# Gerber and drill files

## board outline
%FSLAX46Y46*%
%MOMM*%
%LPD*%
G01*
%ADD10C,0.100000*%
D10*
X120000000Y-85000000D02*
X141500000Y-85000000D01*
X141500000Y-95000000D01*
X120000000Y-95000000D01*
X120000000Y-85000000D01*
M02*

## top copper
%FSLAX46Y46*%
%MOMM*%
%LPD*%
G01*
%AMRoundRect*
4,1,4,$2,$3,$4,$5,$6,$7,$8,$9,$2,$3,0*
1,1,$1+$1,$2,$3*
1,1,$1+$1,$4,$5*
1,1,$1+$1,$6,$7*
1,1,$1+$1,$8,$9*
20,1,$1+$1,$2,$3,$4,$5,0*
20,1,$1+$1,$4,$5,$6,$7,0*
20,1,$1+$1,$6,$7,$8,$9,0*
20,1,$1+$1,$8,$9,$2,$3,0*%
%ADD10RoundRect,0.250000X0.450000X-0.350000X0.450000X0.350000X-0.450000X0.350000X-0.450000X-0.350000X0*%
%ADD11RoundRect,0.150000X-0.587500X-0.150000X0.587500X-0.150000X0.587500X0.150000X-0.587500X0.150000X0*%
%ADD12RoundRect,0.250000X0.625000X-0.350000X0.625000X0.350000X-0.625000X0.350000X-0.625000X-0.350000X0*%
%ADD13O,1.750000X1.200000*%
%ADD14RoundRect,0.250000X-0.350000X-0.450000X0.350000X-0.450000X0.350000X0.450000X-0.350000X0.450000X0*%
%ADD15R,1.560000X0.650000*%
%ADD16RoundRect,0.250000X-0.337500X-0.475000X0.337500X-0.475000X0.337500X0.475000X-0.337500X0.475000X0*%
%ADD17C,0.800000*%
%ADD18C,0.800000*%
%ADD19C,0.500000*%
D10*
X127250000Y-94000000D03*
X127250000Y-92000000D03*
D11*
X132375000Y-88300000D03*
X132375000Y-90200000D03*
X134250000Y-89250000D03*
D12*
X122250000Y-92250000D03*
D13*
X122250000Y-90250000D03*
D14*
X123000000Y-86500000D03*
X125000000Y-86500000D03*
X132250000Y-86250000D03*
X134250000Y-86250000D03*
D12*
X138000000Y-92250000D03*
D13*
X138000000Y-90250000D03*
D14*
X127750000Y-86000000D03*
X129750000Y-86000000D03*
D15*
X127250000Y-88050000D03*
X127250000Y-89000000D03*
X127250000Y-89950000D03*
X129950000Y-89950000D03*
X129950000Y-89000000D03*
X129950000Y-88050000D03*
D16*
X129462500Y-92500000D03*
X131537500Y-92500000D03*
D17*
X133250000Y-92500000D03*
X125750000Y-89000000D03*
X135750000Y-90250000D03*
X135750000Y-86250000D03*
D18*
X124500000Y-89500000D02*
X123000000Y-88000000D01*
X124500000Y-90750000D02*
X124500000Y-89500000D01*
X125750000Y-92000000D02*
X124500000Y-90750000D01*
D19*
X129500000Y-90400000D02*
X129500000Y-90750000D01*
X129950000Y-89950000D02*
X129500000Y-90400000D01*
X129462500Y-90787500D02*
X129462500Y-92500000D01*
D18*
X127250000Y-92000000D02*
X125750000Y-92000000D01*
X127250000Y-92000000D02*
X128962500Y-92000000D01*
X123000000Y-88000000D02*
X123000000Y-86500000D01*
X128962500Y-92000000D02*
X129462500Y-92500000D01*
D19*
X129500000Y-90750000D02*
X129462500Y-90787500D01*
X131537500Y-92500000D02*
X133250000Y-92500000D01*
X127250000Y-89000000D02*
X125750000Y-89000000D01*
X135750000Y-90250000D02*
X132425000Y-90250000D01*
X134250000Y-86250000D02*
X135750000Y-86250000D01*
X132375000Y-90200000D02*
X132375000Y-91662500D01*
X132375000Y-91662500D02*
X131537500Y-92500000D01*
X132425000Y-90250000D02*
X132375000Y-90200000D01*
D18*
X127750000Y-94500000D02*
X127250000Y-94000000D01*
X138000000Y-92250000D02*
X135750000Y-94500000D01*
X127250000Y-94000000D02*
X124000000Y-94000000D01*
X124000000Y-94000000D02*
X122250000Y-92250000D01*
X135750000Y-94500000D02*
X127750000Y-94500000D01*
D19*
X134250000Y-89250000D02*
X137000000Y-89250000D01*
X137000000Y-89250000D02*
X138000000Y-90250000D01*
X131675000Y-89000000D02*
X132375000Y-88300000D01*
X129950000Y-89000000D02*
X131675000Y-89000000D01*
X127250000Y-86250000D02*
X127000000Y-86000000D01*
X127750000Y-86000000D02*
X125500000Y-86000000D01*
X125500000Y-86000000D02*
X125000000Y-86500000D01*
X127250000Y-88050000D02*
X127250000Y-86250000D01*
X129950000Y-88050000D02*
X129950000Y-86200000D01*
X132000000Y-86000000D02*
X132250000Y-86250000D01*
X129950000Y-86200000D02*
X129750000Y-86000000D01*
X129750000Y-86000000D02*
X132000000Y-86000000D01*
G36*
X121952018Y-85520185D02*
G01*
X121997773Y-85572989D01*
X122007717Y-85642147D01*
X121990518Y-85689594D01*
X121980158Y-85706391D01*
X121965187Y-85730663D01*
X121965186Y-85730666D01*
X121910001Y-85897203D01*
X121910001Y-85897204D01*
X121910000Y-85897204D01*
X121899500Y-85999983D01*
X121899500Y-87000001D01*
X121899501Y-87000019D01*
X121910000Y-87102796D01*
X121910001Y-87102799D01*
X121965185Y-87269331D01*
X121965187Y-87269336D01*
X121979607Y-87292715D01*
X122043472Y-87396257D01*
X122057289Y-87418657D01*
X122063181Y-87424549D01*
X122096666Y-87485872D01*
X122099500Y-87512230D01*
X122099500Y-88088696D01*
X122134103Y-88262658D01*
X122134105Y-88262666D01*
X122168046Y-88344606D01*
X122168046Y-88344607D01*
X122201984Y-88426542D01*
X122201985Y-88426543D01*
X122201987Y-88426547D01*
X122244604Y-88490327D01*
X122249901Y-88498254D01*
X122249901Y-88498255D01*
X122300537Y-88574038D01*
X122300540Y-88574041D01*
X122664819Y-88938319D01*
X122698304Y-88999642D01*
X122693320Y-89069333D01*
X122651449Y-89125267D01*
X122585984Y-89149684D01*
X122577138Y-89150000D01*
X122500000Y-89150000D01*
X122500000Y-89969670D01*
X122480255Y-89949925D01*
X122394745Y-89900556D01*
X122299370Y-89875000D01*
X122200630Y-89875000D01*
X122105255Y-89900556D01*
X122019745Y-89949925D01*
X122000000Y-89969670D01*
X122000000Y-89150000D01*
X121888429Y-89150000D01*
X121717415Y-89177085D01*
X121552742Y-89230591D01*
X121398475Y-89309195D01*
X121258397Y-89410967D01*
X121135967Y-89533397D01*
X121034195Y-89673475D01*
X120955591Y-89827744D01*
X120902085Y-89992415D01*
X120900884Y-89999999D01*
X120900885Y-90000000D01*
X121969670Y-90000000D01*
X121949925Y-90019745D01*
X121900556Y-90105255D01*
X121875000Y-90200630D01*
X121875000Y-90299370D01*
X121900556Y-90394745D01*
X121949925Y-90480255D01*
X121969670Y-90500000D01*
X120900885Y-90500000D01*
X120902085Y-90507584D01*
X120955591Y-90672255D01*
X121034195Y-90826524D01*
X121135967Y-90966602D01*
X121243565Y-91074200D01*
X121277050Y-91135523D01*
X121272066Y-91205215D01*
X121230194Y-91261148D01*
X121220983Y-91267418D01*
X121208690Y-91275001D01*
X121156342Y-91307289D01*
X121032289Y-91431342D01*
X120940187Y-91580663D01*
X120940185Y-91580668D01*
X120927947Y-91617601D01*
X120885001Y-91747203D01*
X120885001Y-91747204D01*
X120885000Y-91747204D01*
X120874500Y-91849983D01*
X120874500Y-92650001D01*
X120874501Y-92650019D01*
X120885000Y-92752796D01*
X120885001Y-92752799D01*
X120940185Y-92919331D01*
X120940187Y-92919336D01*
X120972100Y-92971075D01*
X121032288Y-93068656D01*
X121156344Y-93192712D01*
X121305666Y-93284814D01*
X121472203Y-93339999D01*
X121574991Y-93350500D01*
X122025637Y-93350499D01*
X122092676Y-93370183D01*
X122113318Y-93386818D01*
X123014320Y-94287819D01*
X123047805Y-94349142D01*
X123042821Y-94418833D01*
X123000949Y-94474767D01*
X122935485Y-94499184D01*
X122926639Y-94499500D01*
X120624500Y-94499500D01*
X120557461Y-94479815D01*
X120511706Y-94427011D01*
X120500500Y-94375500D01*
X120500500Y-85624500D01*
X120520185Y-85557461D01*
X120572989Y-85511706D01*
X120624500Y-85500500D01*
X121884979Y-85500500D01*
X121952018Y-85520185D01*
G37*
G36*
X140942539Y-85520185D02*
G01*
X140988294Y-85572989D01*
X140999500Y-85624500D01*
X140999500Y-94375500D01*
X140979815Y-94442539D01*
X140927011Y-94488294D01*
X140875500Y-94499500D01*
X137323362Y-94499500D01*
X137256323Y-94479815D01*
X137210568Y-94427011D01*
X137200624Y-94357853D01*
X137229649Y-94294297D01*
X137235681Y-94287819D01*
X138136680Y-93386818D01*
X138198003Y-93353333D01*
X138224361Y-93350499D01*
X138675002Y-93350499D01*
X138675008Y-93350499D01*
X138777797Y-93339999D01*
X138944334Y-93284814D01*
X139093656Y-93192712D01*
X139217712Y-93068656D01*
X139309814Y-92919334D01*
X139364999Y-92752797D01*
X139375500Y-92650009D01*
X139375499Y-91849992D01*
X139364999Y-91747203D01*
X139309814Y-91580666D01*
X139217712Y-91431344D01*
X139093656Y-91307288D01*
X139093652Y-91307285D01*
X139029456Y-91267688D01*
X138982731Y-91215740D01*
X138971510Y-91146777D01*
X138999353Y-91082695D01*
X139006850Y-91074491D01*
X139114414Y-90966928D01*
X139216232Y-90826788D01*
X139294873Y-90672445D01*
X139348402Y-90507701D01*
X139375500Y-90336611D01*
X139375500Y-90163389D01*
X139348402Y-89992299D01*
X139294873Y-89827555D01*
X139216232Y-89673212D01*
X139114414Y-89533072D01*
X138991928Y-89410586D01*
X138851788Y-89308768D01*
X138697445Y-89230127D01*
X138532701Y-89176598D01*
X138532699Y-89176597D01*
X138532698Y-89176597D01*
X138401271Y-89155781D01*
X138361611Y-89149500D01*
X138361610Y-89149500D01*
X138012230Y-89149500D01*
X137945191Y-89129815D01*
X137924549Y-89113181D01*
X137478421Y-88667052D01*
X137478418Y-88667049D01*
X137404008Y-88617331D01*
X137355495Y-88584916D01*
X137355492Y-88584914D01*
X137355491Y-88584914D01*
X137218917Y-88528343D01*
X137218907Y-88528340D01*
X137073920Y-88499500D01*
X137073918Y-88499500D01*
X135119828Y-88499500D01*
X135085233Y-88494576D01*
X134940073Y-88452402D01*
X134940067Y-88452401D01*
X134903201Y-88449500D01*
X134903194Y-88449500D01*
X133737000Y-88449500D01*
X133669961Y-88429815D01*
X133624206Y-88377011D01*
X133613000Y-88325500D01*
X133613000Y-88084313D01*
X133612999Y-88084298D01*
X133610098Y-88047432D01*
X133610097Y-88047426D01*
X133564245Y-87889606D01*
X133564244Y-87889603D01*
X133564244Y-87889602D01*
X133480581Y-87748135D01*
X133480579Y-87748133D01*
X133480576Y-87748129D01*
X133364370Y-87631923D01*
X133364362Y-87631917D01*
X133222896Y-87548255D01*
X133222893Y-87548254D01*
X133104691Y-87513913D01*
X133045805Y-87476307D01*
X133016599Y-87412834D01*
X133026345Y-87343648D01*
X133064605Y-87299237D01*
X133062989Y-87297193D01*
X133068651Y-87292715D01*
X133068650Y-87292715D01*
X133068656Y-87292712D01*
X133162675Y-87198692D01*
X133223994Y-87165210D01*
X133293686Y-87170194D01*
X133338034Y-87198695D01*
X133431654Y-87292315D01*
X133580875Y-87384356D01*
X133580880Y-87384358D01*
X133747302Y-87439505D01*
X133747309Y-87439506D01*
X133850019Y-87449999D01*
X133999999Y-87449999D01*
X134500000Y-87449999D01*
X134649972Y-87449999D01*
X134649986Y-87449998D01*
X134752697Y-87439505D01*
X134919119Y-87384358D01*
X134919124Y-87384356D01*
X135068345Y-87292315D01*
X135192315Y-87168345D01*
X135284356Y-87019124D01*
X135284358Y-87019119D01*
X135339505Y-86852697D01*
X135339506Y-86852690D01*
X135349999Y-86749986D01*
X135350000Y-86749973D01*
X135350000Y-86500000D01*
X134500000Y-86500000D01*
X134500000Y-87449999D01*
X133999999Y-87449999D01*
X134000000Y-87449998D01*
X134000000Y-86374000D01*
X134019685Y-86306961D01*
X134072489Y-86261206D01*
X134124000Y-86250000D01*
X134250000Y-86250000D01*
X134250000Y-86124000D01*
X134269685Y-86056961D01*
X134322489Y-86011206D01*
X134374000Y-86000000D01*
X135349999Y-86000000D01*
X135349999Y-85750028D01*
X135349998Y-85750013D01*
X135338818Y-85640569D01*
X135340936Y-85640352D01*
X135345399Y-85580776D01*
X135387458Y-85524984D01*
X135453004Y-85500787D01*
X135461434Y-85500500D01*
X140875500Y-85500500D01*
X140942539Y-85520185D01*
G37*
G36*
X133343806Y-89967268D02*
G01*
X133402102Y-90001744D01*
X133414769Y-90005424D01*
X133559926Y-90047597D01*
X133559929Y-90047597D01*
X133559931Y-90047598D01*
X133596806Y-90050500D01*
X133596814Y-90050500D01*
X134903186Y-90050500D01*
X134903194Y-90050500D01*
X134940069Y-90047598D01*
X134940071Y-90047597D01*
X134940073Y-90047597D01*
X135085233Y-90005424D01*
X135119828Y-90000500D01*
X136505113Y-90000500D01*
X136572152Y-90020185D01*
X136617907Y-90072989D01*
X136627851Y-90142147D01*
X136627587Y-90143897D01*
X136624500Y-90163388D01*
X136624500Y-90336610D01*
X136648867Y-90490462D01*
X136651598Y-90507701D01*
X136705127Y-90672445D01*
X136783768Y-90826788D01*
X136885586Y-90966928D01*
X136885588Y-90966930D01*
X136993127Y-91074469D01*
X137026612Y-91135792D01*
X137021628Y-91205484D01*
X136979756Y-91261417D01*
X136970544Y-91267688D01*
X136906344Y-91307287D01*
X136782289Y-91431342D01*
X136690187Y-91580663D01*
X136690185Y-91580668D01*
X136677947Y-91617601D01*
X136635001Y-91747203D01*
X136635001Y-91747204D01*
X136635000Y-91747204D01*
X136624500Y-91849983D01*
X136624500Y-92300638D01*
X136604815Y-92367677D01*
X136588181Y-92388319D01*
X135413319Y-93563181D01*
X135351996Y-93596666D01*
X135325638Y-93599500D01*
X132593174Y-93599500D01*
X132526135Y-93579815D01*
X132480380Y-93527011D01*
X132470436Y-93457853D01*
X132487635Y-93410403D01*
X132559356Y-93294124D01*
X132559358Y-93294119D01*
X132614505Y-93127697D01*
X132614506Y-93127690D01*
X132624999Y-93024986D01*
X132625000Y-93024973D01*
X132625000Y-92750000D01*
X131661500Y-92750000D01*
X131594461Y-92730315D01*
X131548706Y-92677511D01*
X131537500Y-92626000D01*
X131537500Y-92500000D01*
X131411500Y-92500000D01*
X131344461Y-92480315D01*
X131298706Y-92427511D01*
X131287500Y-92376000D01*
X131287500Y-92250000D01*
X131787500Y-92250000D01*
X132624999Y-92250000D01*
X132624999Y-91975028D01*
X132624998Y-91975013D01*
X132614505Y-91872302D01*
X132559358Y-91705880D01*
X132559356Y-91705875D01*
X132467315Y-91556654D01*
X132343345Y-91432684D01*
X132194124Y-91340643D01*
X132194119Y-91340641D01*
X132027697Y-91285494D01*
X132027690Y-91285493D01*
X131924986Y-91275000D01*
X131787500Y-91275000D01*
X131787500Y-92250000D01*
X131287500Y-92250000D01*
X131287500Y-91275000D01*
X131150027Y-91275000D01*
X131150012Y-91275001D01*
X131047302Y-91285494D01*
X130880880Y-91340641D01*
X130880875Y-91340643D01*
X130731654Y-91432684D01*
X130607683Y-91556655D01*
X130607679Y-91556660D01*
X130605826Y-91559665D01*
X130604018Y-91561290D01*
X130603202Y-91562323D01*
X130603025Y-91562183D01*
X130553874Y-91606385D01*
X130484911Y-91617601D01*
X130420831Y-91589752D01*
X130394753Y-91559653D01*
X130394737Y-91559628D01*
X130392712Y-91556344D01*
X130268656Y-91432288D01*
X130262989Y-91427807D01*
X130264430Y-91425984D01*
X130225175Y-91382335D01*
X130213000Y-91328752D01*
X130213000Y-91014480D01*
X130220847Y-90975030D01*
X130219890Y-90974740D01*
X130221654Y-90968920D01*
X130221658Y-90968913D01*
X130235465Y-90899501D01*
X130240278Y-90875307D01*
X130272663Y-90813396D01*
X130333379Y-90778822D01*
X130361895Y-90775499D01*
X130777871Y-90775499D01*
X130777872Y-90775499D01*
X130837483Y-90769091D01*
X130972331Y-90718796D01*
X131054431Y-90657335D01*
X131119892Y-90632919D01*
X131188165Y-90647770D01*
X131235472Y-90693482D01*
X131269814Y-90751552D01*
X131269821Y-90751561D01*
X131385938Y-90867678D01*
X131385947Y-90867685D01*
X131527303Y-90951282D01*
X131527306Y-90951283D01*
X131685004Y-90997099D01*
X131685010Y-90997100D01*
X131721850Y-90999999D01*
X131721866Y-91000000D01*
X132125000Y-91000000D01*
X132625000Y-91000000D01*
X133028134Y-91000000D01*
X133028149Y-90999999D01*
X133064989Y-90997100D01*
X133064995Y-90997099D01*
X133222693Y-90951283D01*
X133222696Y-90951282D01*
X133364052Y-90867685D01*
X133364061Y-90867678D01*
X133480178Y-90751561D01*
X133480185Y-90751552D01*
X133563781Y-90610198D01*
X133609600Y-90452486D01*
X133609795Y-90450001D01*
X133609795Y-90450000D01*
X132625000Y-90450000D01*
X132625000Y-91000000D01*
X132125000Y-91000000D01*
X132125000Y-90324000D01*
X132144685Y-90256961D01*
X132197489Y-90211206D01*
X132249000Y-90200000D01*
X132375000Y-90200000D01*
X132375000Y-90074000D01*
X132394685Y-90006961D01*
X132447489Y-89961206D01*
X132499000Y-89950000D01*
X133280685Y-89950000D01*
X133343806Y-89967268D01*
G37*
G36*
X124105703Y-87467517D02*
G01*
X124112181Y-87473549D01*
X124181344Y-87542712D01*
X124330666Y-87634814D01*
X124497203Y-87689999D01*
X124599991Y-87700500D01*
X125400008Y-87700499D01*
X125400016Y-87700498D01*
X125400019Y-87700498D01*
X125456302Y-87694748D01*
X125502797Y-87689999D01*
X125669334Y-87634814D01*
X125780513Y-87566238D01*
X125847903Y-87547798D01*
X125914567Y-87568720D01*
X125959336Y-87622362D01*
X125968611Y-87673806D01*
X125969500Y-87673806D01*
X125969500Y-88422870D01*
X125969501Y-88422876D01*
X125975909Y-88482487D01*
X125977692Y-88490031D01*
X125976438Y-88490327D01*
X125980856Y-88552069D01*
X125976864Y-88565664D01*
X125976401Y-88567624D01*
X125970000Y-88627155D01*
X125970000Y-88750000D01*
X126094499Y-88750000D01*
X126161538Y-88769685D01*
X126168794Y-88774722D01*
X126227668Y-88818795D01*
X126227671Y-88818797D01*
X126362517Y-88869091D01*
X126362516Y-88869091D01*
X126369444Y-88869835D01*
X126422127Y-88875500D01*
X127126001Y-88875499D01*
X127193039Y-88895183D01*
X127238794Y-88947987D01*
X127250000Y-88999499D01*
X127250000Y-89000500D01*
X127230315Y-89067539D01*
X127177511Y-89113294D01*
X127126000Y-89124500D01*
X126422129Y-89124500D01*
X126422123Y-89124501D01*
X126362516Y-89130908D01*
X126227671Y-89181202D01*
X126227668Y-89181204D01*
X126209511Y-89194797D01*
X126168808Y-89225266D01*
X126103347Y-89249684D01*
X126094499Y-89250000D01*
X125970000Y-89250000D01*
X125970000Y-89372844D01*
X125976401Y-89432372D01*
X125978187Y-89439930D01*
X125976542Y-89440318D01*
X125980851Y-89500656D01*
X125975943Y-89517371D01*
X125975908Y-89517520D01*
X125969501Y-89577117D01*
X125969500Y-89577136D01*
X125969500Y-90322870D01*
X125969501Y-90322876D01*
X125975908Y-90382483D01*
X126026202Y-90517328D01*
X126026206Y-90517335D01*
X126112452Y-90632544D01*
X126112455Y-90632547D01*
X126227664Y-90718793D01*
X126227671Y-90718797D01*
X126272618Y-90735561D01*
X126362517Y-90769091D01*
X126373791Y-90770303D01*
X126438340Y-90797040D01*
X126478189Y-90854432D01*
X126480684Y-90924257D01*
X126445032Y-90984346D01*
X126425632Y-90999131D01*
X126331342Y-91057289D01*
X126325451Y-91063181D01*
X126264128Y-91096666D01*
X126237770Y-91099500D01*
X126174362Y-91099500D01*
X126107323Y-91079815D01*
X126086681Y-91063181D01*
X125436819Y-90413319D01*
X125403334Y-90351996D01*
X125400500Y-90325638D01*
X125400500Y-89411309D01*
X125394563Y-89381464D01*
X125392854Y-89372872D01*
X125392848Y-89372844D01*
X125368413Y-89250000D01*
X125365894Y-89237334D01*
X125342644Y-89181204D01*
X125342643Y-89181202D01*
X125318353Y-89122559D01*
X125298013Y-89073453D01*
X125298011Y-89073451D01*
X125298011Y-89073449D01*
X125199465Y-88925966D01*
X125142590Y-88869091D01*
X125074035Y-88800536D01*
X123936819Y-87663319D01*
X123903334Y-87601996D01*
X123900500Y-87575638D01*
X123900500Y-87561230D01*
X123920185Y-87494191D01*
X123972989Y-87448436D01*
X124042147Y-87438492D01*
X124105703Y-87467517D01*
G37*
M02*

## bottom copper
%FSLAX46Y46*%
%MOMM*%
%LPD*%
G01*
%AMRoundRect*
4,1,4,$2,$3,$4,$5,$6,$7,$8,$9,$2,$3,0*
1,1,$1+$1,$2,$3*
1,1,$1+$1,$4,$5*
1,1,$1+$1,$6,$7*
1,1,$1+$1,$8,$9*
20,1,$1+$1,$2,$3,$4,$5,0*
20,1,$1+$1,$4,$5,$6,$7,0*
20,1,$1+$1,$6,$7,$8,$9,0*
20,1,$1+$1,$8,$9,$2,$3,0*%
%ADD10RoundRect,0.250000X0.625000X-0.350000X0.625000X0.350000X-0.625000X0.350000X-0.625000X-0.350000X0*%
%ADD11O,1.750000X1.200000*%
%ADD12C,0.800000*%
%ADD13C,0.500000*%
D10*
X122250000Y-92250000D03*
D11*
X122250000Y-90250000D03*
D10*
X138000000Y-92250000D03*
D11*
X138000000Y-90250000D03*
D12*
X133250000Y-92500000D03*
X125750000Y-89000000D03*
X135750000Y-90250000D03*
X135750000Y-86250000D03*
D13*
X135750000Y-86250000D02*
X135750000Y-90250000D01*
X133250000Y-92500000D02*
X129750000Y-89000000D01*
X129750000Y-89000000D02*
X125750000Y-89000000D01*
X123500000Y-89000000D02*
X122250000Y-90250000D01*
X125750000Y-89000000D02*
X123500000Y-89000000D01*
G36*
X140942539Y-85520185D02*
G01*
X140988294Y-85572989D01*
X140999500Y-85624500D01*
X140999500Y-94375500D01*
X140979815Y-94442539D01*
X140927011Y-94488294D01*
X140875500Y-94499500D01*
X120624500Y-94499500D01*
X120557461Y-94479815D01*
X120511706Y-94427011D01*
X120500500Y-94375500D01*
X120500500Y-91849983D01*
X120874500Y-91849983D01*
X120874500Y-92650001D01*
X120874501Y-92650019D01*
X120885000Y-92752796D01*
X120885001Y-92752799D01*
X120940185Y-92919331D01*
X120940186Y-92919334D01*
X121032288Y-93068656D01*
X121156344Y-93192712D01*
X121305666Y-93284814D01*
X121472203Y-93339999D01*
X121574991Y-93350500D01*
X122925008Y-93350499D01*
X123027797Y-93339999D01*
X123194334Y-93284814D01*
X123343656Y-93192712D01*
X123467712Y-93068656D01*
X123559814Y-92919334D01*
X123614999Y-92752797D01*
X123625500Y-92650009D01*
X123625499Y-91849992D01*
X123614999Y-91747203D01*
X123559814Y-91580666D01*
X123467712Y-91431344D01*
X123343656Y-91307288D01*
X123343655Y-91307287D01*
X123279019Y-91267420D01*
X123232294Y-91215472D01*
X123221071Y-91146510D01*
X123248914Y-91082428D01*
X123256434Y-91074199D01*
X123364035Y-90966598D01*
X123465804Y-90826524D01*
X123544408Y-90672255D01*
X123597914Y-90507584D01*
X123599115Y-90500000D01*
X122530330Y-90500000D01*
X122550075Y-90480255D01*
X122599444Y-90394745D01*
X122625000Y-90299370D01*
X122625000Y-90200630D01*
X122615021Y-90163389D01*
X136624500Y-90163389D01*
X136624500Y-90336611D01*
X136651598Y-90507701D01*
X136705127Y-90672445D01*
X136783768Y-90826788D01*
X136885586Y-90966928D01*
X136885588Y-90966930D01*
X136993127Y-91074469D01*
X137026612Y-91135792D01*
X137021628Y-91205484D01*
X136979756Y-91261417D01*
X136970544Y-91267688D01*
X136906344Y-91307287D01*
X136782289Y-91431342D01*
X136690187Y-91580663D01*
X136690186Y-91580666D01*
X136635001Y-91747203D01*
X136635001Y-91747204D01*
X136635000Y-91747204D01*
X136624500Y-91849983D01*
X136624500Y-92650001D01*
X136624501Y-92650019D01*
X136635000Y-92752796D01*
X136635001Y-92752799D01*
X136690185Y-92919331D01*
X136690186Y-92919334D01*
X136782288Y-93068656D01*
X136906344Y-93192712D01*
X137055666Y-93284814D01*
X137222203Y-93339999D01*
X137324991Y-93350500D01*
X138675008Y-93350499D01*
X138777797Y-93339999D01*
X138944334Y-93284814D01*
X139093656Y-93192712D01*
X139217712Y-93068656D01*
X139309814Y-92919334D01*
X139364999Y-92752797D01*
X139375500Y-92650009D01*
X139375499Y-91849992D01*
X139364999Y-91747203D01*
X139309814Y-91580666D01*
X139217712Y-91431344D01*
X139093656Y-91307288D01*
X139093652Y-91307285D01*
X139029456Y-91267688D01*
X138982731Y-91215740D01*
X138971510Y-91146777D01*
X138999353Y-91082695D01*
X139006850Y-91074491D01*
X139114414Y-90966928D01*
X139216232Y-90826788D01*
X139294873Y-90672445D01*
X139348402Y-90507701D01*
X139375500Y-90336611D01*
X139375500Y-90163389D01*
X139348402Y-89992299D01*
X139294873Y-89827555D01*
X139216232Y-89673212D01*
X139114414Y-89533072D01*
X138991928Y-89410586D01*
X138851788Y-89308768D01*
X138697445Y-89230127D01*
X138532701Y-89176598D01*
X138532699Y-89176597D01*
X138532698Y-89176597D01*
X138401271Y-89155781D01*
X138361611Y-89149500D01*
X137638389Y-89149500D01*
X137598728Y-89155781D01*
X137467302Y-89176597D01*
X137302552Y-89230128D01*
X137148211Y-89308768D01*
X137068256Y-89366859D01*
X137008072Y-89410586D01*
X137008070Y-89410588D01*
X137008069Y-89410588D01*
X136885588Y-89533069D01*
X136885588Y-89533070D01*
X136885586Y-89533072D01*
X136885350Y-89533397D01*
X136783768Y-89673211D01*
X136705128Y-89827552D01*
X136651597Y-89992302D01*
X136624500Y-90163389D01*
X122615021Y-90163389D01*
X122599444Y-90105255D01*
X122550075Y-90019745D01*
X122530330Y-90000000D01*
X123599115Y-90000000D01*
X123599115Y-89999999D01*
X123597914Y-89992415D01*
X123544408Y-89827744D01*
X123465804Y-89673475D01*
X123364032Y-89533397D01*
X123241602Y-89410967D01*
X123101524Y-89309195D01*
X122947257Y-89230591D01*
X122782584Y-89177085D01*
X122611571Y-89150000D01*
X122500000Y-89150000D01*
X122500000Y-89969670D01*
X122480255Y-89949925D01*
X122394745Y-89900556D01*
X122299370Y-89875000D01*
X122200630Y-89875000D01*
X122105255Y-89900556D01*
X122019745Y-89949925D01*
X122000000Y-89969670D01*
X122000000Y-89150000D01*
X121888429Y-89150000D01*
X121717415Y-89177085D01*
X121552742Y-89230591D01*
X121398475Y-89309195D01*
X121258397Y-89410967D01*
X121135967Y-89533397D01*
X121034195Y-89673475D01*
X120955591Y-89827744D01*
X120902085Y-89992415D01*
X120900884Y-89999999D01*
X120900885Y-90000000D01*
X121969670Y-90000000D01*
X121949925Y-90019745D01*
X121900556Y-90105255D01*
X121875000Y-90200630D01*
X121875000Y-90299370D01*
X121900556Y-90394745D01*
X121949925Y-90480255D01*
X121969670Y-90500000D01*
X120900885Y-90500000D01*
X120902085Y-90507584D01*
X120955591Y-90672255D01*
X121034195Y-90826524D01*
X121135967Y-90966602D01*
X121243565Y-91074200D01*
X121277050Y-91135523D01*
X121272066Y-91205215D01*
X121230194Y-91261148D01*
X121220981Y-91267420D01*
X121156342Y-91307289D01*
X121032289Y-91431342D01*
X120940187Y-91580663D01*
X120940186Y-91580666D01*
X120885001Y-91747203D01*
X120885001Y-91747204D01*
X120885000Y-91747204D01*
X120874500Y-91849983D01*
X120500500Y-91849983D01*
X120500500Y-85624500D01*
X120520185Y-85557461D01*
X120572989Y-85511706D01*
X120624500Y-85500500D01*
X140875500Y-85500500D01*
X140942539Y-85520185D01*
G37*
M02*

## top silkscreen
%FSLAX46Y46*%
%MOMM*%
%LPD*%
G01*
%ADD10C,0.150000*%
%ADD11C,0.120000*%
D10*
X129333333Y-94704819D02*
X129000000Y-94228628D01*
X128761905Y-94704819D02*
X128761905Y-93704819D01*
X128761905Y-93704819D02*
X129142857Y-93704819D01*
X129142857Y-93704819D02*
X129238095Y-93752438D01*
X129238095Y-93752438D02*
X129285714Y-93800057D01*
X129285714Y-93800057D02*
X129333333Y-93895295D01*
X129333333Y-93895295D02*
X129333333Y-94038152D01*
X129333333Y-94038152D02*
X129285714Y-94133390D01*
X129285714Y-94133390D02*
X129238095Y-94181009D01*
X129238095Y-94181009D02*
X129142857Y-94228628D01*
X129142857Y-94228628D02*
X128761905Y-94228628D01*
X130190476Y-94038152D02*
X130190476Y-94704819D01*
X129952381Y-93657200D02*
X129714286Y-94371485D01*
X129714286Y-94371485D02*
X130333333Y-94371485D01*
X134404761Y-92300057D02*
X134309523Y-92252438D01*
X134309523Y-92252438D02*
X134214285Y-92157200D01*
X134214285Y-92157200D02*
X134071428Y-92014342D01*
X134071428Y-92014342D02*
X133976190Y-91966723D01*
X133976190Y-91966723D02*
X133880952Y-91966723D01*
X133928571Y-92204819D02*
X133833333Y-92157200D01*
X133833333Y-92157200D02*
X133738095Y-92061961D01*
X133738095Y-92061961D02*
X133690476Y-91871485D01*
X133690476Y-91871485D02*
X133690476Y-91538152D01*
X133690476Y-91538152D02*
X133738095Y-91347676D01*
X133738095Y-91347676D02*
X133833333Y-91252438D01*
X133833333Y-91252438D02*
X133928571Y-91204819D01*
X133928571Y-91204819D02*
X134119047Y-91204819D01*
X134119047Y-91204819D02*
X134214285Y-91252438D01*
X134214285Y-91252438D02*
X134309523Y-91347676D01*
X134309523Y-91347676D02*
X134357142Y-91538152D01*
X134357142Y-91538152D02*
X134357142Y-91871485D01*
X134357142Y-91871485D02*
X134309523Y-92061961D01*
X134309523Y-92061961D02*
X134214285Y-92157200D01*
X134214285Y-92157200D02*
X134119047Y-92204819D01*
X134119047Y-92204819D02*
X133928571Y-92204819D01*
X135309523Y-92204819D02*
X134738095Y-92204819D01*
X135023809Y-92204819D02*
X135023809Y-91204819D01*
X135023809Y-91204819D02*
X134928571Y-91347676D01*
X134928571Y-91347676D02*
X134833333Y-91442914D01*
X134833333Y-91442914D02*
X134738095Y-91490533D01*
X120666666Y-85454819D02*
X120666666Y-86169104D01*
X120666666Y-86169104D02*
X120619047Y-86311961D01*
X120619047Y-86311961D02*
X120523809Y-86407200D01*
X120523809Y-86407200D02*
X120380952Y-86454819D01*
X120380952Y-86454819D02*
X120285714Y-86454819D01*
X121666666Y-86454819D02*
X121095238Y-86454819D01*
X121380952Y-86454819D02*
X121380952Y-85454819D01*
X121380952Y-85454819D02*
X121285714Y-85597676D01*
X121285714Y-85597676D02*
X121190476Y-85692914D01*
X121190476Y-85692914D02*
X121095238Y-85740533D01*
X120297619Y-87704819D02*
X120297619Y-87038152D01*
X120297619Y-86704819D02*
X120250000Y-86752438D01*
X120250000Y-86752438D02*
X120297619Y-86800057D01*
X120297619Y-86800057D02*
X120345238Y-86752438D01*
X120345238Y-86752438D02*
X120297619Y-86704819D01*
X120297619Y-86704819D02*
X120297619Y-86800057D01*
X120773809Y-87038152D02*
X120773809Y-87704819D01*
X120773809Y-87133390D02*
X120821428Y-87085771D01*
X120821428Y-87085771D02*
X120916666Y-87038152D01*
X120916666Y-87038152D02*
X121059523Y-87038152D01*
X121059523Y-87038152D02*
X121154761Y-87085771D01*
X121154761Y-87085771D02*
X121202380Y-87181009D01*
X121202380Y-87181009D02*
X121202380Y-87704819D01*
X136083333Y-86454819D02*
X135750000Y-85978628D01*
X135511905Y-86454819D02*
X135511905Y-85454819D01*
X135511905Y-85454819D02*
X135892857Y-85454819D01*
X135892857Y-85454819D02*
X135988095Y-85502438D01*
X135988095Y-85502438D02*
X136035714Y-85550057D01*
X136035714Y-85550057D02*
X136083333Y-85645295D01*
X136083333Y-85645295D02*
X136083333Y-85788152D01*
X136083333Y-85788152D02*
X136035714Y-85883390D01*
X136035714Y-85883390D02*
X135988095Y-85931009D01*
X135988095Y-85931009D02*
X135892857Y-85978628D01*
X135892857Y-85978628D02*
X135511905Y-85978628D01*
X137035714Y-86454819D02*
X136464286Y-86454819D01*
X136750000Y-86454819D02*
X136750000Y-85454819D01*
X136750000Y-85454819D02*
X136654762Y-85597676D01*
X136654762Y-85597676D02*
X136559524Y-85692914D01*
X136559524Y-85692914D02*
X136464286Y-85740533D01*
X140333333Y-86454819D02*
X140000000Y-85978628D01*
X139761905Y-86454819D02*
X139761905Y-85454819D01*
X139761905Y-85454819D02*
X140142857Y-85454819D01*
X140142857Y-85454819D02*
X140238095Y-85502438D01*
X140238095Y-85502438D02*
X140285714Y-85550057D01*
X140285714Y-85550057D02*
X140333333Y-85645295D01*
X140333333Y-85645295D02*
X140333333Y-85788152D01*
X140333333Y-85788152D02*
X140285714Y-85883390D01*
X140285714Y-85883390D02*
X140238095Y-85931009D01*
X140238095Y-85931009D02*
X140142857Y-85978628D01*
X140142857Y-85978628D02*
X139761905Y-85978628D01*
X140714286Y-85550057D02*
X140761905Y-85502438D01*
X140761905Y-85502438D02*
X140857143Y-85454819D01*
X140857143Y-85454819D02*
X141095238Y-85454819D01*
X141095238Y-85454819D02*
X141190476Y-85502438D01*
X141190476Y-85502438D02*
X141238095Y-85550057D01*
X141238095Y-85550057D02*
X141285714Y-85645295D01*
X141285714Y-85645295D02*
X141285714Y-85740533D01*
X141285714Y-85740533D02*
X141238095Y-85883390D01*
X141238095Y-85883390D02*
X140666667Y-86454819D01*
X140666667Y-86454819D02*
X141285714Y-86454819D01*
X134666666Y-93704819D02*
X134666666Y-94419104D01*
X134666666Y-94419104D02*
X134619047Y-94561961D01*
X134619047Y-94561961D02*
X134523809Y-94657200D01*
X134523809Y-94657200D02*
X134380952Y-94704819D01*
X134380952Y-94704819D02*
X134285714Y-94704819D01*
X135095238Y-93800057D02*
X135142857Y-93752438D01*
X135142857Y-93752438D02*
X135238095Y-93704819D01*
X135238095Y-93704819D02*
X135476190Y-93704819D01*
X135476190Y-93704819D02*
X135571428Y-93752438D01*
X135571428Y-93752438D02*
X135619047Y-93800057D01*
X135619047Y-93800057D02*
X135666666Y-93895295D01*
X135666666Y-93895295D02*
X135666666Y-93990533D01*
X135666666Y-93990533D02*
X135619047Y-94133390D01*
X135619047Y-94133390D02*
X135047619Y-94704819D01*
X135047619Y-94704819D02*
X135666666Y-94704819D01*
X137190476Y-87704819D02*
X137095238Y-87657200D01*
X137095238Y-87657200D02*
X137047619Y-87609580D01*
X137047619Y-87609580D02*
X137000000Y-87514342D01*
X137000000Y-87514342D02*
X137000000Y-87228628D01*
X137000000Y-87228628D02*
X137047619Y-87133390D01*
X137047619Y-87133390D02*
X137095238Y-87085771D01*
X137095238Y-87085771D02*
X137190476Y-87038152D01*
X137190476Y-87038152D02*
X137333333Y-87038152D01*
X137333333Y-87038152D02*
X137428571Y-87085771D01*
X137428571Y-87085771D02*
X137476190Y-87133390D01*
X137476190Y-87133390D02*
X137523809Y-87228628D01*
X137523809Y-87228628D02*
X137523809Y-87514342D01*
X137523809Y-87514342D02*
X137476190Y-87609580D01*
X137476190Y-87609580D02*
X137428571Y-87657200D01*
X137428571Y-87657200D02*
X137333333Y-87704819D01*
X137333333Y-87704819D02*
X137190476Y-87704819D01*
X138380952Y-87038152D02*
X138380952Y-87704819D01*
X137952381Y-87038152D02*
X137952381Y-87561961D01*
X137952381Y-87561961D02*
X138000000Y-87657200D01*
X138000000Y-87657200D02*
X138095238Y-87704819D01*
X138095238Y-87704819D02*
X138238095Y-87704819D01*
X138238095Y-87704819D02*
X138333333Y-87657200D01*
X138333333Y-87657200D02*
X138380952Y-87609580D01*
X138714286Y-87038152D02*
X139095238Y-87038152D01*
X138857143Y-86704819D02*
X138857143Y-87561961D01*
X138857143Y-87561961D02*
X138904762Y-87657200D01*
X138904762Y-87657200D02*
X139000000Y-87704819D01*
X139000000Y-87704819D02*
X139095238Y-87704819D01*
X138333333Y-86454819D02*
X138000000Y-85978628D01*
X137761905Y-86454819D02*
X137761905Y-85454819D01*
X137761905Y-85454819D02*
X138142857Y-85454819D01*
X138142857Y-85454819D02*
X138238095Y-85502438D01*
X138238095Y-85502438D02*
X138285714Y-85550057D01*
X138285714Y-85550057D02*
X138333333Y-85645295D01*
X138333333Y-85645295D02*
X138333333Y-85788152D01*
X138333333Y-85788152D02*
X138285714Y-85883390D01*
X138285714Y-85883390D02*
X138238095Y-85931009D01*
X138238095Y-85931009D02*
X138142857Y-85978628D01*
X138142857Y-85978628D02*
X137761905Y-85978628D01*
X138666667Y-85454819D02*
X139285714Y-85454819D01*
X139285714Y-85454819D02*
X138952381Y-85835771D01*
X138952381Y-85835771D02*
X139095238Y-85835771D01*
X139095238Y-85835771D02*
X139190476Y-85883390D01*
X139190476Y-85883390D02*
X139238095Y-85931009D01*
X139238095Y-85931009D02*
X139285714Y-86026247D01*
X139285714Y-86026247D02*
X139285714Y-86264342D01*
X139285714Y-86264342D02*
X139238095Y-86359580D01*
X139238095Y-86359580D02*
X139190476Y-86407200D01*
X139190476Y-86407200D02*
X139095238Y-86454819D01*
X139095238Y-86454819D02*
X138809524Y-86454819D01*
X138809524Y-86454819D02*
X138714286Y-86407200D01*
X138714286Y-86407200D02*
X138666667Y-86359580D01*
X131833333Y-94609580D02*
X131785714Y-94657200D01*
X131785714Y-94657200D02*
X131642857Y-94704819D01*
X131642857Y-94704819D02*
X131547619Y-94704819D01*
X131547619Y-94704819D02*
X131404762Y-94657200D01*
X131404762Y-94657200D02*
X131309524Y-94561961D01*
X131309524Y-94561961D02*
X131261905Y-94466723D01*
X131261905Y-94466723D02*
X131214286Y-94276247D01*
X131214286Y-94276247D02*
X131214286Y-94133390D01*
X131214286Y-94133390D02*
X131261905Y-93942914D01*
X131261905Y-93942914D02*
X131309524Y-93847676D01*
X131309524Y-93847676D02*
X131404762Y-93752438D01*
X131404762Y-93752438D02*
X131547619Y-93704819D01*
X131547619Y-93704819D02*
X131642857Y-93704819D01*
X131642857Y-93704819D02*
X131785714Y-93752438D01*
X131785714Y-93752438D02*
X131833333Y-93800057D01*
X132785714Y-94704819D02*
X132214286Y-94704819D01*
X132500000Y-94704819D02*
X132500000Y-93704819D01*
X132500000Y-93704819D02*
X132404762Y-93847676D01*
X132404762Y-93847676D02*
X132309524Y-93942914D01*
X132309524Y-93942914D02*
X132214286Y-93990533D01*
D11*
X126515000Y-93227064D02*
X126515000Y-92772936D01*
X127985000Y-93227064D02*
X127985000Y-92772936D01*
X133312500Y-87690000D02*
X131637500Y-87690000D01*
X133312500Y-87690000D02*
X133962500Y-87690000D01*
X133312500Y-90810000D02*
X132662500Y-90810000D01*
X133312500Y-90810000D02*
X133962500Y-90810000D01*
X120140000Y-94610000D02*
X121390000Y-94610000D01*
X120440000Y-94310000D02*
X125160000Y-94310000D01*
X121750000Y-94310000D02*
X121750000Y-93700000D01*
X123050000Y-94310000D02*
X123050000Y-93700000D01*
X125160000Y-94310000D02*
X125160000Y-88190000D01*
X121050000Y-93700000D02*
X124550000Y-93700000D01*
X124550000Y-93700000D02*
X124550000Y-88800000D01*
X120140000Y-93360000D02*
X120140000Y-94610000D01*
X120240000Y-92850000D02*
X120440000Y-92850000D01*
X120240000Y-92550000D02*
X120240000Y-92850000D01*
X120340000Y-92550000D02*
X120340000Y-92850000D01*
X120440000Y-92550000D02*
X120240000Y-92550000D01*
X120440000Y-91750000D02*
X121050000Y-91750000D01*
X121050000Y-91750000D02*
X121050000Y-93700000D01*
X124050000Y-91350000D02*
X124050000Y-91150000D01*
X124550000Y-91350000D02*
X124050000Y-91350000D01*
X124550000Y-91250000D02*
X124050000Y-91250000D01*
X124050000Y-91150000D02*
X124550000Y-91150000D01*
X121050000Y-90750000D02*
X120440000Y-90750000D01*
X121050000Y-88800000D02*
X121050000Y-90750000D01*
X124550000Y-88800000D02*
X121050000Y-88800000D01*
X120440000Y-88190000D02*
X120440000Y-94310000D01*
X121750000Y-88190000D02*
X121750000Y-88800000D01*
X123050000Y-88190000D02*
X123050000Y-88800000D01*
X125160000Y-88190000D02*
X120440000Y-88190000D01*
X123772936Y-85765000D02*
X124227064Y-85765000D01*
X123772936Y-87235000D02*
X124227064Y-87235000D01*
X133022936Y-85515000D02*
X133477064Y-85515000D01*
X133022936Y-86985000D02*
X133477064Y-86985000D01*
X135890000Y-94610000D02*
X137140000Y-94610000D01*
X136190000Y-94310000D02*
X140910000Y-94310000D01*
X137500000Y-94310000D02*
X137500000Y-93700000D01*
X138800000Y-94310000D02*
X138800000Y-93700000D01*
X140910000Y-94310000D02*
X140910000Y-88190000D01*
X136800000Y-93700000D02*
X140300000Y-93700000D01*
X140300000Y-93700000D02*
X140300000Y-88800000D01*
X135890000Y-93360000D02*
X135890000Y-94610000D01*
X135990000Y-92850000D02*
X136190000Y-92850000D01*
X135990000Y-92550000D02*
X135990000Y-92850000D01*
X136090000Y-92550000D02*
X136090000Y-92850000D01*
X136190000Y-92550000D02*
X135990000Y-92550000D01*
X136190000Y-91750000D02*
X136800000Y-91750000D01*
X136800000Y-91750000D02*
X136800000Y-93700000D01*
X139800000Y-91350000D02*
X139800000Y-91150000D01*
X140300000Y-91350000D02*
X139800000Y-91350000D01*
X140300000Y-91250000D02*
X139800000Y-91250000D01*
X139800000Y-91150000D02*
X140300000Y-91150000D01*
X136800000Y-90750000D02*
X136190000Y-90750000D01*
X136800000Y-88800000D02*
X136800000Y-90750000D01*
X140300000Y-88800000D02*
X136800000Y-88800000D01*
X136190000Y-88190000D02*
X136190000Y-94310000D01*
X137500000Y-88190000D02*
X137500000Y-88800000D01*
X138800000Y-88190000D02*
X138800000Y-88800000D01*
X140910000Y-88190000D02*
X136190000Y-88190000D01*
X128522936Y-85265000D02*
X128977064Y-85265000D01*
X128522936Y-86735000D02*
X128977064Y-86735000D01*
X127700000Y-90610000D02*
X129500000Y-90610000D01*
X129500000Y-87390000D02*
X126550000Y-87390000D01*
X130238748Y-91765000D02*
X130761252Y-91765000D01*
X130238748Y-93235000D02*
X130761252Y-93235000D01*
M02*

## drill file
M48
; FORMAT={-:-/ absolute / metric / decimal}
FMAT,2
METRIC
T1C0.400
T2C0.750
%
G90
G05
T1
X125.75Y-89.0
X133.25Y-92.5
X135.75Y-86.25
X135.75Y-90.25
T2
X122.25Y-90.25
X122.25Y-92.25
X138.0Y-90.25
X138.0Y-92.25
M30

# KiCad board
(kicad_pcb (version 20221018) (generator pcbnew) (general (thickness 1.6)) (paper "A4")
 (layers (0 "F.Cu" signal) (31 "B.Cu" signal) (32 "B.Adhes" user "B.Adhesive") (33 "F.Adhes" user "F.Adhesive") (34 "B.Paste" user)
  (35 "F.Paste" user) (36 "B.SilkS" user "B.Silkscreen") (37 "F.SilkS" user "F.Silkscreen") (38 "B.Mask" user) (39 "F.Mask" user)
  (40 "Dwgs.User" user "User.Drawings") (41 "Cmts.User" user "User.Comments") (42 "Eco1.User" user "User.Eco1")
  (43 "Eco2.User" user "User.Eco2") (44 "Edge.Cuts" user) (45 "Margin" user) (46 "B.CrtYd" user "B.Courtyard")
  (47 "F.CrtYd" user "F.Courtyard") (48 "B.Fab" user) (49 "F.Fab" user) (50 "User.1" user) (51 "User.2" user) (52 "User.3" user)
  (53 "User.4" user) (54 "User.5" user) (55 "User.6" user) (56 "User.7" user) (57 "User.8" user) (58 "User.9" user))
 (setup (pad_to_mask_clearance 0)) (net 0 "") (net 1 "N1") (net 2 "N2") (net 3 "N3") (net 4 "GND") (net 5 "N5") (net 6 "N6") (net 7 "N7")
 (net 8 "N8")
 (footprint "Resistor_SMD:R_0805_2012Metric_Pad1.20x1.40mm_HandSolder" (layer "F.Cu") (at 127.25 93 90)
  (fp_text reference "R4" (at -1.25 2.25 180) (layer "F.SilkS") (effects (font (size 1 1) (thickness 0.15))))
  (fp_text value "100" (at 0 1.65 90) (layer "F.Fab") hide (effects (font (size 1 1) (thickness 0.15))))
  (fp_line (start -0.227064 -0.735) (end 0.227064 -0.735) (stroke (width 0.12) (type solid)) (layer "F.SilkS"))
  (fp_line (start -0.227064 0.735) (end 0.227064 0.735) (stroke (width 0.12) (type solid)) (layer "F.SilkS"))
  (pad "1" smd roundrect (at -1 0 90) (size 1.2 1.4) (layers "F.Cu" "F.Paste" "F.Mask") (roundrect_rratio 0.2083333333) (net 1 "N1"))
  (pad "2" smd roundrect (at 1 0 90) (size 1.2 1.4) (layers "F.Cu" "F.Paste" "F.Mask") (roundrect_rratio 0.2083333333) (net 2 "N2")))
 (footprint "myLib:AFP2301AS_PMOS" (layer "F.Cu") (at 133.3125 89.25)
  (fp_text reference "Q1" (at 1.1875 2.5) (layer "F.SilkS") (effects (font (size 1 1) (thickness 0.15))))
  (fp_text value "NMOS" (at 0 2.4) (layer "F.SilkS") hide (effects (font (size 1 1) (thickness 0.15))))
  (fp_line (start 0 -1.56) (end -1.675 -1.56) (stroke (width 0.12) (type solid)) (layer "F.SilkS"))
  (fp_line (start 0 -1.56) (end 0.65 -1.56) (stroke (width 0.12) (type solid)) (layer "F.SilkS"))
  (fp_line (start 0 1.56) (end -0.65 1.56) (stroke (width 0.12) (type solid)) (layer "F.SilkS"))
  (fp_line (start 0 1.56) (end 0.65 1.56) (stroke (width 0.12) (type solid)) (layer "F.SilkS"))
  (pad "1" smd roundrect (at -0.9375 -0.95) (size 1.475 0.6) (layers "F.Cu" "F.Paste" "F.Mask") (roundrect_rratio 0.25) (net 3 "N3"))
  (pad "2" smd roundrect (at -0.9375 0.95) (size 1.475 0.6) (layers "F.Cu" "F.Paste" "F.Mask") (roundrect_rratio 0.25) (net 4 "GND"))
  (pad "3" smd roundrect (at 0.9375 0) (size 1.475 0.6) (layers "F.Cu" "F.Paste" "F.Mask") (roundrect_rratio 0.25) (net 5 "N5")))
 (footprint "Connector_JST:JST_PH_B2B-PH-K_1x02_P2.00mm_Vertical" (layer "F.Cu") (at 122.25 92.25 90)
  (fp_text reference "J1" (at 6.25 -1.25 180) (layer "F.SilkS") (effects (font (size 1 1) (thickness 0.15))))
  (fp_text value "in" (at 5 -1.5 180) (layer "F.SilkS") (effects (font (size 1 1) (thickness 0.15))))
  (fp_line (start -2.36 -2.11) (end -2.36 -0.86) (stroke (width 0.12) (type solid)) (layer "F.SilkS"))
  (fp_line (start -2.06 -1.81) (end -2.06 2.91) (stroke (width 0.12) (type solid)) (layer "F.SilkS"))
  (fp_line (start -2.06 -0.5) (end -1.45 -0.5) (stroke (width 0.12) (type solid)) (layer "F.SilkS"))
  (fp_line (start -2.06 0.8) (end -1.45 0.8) (stroke (width 0.12) (type solid)) (layer "F.SilkS"))
  (fp_line (start -2.06 2.91) (end 4.06 2.91) (stroke (width 0.12) (type solid)) (layer "F.SilkS"))
  (fp_line (start -1.45 -1.2) (end -1.45 2.3) (stroke (width 0.12) (type solid)) (layer "F.SilkS"))
  (fp_line (start -1.45 2.3) (end 3.45 2.3) (stroke (width 0.12) (type solid)) (layer "F.SilkS"))
  (fp_line (start -1.11 -2.11) (end -2.36 -2.11) (stroke (width 0.12) (type solid)) (layer "F.SilkS"))
  (fp_line (start -0.6 -2.01) (end -0.6 -1.81) (stroke (width 0.12) (type solid)) (layer "F.SilkS"))
  (fp_line (start -0.3 -2.01) (end -0.6 -2.01) (stroke (width 0.12) (type solid)) (layer "F.SilkS"))
  (fp_line (start -0.3 -1.91) (end -0.6 -1.91) (stroke (width 0.12) (type solid)) (layer "F.SilkS"))
  (fp_line (start -0.3 -1.81) (end -0.3 -2.01) (stroke (width 0.12) (type solid)) (layer "F.SilkS"))
  (fp_line (start 0.5 -1.81) (end 0.5 -1.2) (stroke (width 0.12) (type solid)) (layer "F.SilkS"))
  (fp_line (start 0.5 -1.2) (end -1.45 -1.2) (stroke (width 0.12) (type solid)) (layer "F.SilkS"))
  (fp_line (start 0.9 1.8) (end 1.1 1.8) (stroke (width 0.12) (type solid)) (layer "F.SilkS"))
  (fp_line (start 0.9 2.3) (end 0.9 1.8) (stroke (width 0.12) (type solid)) (layer "F.SilkS"))
  (fp_line (start 1 2.3) (end 1 1.8) (stroke (width 0.12) (type solid)) (layer "F.SilkS"))
  (fp_line (start 1.1 1.8) (end 1.1 2.3) (stroke (width 0.12) (type solid)) (layer "F.SilkS"))
  (fp_line (start 1.5 -1.2) (end 1.5 -1.81) (stroke (width 0.12) (type solid)) (layer "F.SilkS"))
  (fp_line (start 3.45 -1.2) (end 1.5 -1.2) (stroke (width 0.12) (type solid)) (layer "F.SilkS"))
  (fp_line (start 3.45 2.3) (end 3.45 -1.2) (stroke (width 0.12) (type solid)) (layer "F.SilkS"))
  (fp_line (start 4.06 -1.81) (end -2.06 -1.81) (stroke (width 0.12) (type solid)) (layer "F.SilkS"))
  (fp_line (start 4.06 -0.5) (end 3.45 -0.5) (stroke (width 0.12) (type solid)) (layer "F.SilkS"))
  (fp_line (start 4.06 0.8) (end 3.45 0.8) (stroke (width 0.12) (type solid)) (layer "F.SilkS"))
  (fp_line (start 4.06 2.91) (end 4.06 -1.81) (stroke (width 0.12) (type solid)) (layer "F.SilkS"))
  (pad "1" thru_hole roundrect (at 0 0 90) (size 1.2 1.75) (drill 0.75) (layers "*.Cu" "*.Mask") (roundrect_rratio 0.2083333333)
   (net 1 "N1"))
  (pad "2" thru_hole oval (at 2 0 90) (size 1.2 1.75) (drill 0.75) (layers "*.Cu" "*.Mask") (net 4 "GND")))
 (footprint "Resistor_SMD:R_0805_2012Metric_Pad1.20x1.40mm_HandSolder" (layer "F.Cu") (at 124 86.5)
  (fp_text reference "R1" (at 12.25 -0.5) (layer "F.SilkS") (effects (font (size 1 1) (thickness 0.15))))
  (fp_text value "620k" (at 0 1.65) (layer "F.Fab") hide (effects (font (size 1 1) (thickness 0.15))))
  (fp_line (start -0.227064 -0.735) (end 0.227064 -0.735) (stroke (width 0.12) (type solid)) (layer "F.SilkS"))
  (fp_line (start -0.227064 0.735) (end 0.227064 0.735) (stroke (width 0.12) (type solid)) (layer "F.SilkS"))
  (pad "1" smd roundrect (at -1 0) (size 1.2 1.4) (layers "F.Cu" "F.Paste" "F.Mask") (roundrect_rratio 0.2083333333) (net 2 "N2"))
  (pad "2" smd roundrect (at 1 0) (size 1.2 1.4) (layers "F.Cu" "F.Paste" "F.Mask") (roundrect_rratio 0.2083333333) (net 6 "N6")))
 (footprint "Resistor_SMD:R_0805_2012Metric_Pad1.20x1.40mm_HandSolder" (layer "F.Cu") (at 133.25 86.25)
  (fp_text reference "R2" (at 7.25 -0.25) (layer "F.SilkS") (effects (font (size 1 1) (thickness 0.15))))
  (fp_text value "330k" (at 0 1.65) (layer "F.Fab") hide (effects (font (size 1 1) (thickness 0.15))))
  (fp_line (start -0.227064 -0.735) (end 0.227064 -0.735) (stroke (width 0.12) (type solid)) (layer "F.SilkS"))
  (fp_line (start -0.227064 0.735) (end 0.227064 0.735) (stroke (width 0.12) (type solid)) (layer "F.SilkS"))
  (pad "1" smd roundrect (at -1 0) (size 1.2 1.4) (layers "F.Cu" "F.Paste" "F.Mask") (roundrect_rratio 0.2083333333) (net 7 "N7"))
  (pad "2" smd roundrect (at 1 0) (size 1.2 1.4) (layers "F.Cu" "F.Paste" "F.Mask") (roundrect_rratio 0.2083333333) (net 4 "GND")))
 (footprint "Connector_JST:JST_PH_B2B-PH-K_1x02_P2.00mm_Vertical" (layer "F.Cu") (at 138 92.25 90)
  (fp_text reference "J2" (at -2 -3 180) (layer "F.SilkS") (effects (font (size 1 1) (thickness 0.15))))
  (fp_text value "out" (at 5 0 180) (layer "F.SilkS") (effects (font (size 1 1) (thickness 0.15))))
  (fp_line (start -2.36 -2.11) (end -2.36 -0.86) (stroke (width 0.12) (type solid)) (layer "F.SilkS"))
  (fp_line (start -2.06 -1.81) (end -2.06 2.91) (stroke (width 0.12) (type solid)) (layer "F.SilkS"))
  (fp_line (start -2.06 -0.5) (end -1.45 -0.5) (stroke (width 0.12) (type solid)) (layer "F.SilkS"))
  (fp_line (start -2.06 0.8) (end -1.45 0.8) (stroke (width 0.12) (type solid)) (layer "F.SilkS"))
  (fp_line (start -2.06 2.91) (end 4.06 2.91) (stroke (width 0.12) (type solid)) (layer "F.SilkS"))
  (fp_line (start -1.45 -1.2) (end -1.45 2.3) (stroke (width 0.12) (type solid)) (layer "F.SilkS"))
  (fp_line (start -1.45 2.3) (end 3.45 2.3) (stroke (width 0.12) (type solid)) (layer "F.SilkS"))
  (fp_line (start -1.11 -2.11) (end -2.36 -2.11) (stroke (width 0.12) (type solid)) (layer "F.SilkS"))
  (fp_line (start -0.6 -2.01) (end -0.6 -1.81) (stroke (width 0.12) (type solid)) (layer "F.SilkS"))
  (fp_line (start -0.3 -2.01) (end -0.6 -2.01) (stroke (width 0.12) (type solid)) (layer "F.SilkS"))
  (fp_line (start -0.3 -1.91) (end -0.6 -1.91) (stroke (width 0.12) (type solid)) (layer "F.SilkS"))
  (fp_line (start -0.3 -1.81) (end -0.3 -2.01) (stroke (width 0.12) (type solid)) (layer "F.SilkS"))
  (fp_line (start 0.5 -1.81) (end 0.5 -1.2) (stroke (width 0.12) (type solid)) (layer "F.SilkS"))
  (fp_line (start 0.5 -1.2) (end -1.45 -1.2) (stroke (width 0.12) (type solid)) (layer "F.SilkS"))
  (fp_line (start 0.9 1.8) (end 1.1 1.8) (stroke (width 0.12) (type solid)) (layer "F.SilkS"))
  (fp_line (start 0.9 2.3) (end 0.9 1.8) (stroke (width 0.12) (type solid)) (layer "F.SilkS"))
  (fp_line (start 1 2.3) (end 1 1.8) (stroke (width 0.12) (type solid)) (layer "F.SilkS"))
  (fp_line (start 1.1 1.8) (end 1.1 2.3) (stroke (width 0.12) (type solid)) (layer "F.SilkS"))
  (fp_line (start 1.5 -1.2) (end 1.5 -1.81) (stroke (width 0.12) (type solid)) (layer "F.SilkS"))
  (fp_line (start 3.45 -1.2) (end 1.5 -1.2) (stroke (width 0.12) (type solid)) (layer "F.SilkS"))
  (fp_line (start 3.45 2.3) (end 3.45 -1.2) (stroke (width 0.12) (type solid)) (layer "F.SilkS"))
  (fp_line (start 4.06 -1.81) (end -2.06 -1.81) (stroke (width 0.12) (type solid)) (layer "F.SilkS"))
  (fp_line (start 4.06 -0.5) (end 3.45 -0.5) (stroke (width 0.12) (type solid)) (layer "F.SilkS"))
  (fp_line (start 4.06 0.8) (end 3.45 0.8) (stroke (width 0.12) (type solid)) (layer "F.SilkS"))
  (fp_line (start 4.06 2.91) (end 4.06 -1.81) (stroke (width 0.12) (type solid)) (layer "F.SilkS"))
  (pad "1" thru_hole roundrect (at 0 0 90) (size 1.2 1.75) (drill 0.75) (layers "*.Cu" "*.Mask") (roundrect_rratio 0.2083333333)
   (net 1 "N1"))
  (pad "2" thru_hole oval (at 2 0 90) (size 1.2 1.75) (drill 0.75) (layers "*.Cu" "*.Mask") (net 5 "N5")))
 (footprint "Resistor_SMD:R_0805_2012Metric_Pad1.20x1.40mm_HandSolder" (layer "F.Cu") (at 128.75 86)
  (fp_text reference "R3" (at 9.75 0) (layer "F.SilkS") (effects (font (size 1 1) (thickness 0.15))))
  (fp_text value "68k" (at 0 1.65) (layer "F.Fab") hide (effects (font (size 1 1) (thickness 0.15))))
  (fp_line (start -0.227064 -0.735) (end 0.227064 -0.735) (stroke (width 0.12) (type solid)) (layer "F.SilkS"))
  (fp_line (start -0.227064 0.735) (end 0.227064 0.735) (stroke (width 0.12) (type solid)) (layer "F.SilkS"))
  (pad "1" smd roundrect (at -1 0) (size 1.2 1.4) (layers "F.Cu" "F.Paste" "F.Mask") (roundrect_rratio 0.2083333333) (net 6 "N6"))
  (pad "2" smd roundrect (at 1 0) (size 1.2 1.4) (layers "F.Cu" "F.Paste" "F.Mask") (roundrect_rratio 0.2083333333) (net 7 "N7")))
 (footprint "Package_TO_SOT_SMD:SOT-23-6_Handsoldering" (layer "F.Cu") (at 128.6 89)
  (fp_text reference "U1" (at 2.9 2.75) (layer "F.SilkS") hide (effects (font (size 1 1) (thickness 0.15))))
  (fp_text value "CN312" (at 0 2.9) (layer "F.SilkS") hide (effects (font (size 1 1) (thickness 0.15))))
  (fp_line (start -0.9 1.61) (end 0.9 1.61) (stroke (width 0.12) (type solid)) (layer "F.SilkS"))
  (fp_line (start 0.9 -1.61) (end -2.05 -1.61) (stroke (width 0.12) (type solid)) (layer "F.SilkS"))
  (pad "1" smd rect (at -1.35 -0.95) (size 1.56 0.65) (layers "F.Cu" "F.Paste" "F.Mask") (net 6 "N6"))
  (pad "2" smd rect (at -1.35 0) (size 1.56 0.65) (layers "F.Cu" "F.Paste" "F.Mask") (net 4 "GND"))
  (pad "3" smd rect (at -1.35 0.95) (size 1.56 0.65) (layers "F.Cu" "F.Paste" "F.Mask") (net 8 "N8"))
  (pad "4" smd rect (at 1.35 0.95) (size 1.56 0.65) (layers "F.Cu" "F.Paste" "F.Mask") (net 2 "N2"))
  (pad "5" smd rect (at 1.35 0) (size 1.56 0.65) (layers "F.Cu" "F.Paste" "F.Mask") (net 3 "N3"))
  (pad "6" smd rect (at 1.35 -0.95) (size 1.56 0.65) (layers "F.Cu" "F.Paste" "F.Mask") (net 7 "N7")))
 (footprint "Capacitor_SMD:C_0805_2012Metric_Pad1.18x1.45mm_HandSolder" (layer "F.Cu") (at 130.5 92.5)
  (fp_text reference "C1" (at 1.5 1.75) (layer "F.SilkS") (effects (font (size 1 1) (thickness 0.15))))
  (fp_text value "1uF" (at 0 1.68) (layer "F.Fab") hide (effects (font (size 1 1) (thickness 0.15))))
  (fp_line (start -0.261252 -0.735) (end 0.261252 -0.735) (stroke (width 0.12) (type solid)) (layer "F.SilkS"))
  (fp_line (start -0.261252 0.735) (end 0.261252 0.735) (stroke (width 0.12) (type solid)) (layer "F.SilkS"))
  (pad "1" smd roundrect (at -1.0375 0) (size 1.175 1.45) (layers "F.Cu" "F.Paste" "F.Mask") (roundrect_rratio 0.2127659574) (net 2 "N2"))
  (pad "2" smd roundrect (at 1.0375 0) (size 1.175 1.45) (layers "F.Cu" "F.Paste" "F.Mask") (roundrect_rratio 0.2127659574) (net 4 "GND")))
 (gr_rect (start 120 85) (end 141.5 95) (stroke (width 0.1) (type default)) (fill none) (layer "Edge.Cuts"))
 (segment (start 124.5 89.5) (end 123 88) (width 0.8) (layer "F.Cu") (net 2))
 (segment (start 124.5 90.75) (end 124.5 89.5) (width 0.8) (layer "F.Cu") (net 2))
 (segment (start 125.75 92) (end 124.5 90.75) (width 0.8) (layer "F.Cu") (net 2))
 (segment (start 129.5 90.4) (end 129.5 90.75) (width 0.5) (layer "F.Cu") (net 2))
 (segment (start 129.95 89.95) (end 129.5 90.4) (width 0.5) (layer "F.Cu") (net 2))
 (segment (start 129.4625 90.7875) (end 129.4625 92.5) (width 0.5) (layer "F.Cu") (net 2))
 (segment (start 127.25 92) (end 125.75 92) (width 0.8) (layer "F.Cu") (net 2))
 (segment (start 127.25 92) (end 128.9625 92) (width 0.8) (layer "F.Cu") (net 2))
 (segment (start 123 88) (end 123 86.5) (width 0.8) (layer "F.Cu") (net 2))
 (segment (start 128.9625 92) (end 129.4625 92.5) (width 0.8) (layer "F.Cu") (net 2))
 (segment (start 129.5 90.75) (end 129.4625 90.7875) (width 0.5) (layer "F.Cu") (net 2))
 (segment (start 131.5375 92.5) (end 133.25 92.5) (width 0.5) (layer "F.Cu") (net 4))
 (segment (start 127.25 89) (end 125.75 89) (width 0.5) (layer "F.Cu") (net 4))
 (segment (start 135.75 90.25) (end 132.425 90.25) (width 0.5) (layer "F.Cu") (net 4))
 (segment (start 134.25 86.25) (end 135.75 86.25) (width 0.5) (layer "F.Cu") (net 4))
 (segment (start 132.375 90.2) (end 132.375 91.6625) (width 0.5) (layer "F.Cu") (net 4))
 (segment (start 132.375 91.6625) (end 131.5375 92.5) (width 0.5) (layer "F.Cu") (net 4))
 (segment (start 132.425 90.25) (end 132.375 90.2) (width 0.5) (layer "F.Cu") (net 4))
 (via (at 133.25 92.5) (size 0.8) (drill 0.4) (layers "F.Cu" "B.Cu") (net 4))
 (via (at 125.75 89) (size 0.8) (drill 0.4) (layers "F.Cu" "B.Cu") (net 4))
 (via (at 135.75 90.25) (size 0.8) (drill 0.4) (layers "F.Cu" "B.Cu") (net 4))
 (via (at 135.75 86.25) (size 0.8) (drill 0.4) (layers "F.Cu" "B.Cu") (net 4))
 (segment (start 135.75 86.25) (end 135.75 90.25) (width 0.5) (layer "B.Cu") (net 4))
 (segment (start 133.25 92.5) (end 129.75 89) (width 0.5) (layer "B.Cu") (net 4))
 (segment (start 129.75 89) (end 125.75 89) (width 0.5) (layer "B.Cu") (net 4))
 (segment (start 123.5 89) (end 122.25 90.25) (width 0.5) (layer "B.Cu") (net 4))
 (segment (start 125.75 89) (end 123.5 89) (width 0.5) (layer "B.Cu") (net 4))
 (segment (start 127.75 94.5) (end 127.25 94) (width 0.8) (layer "F.Cu") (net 1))
 (segment (start 138 92.25) (end 135.75 94.5) (width 0.8) (layer "F.Cu") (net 1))
 (segment (start 127.25 94) (end 124 94) (width 0.8) (layer "F.Cu") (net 1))
 (segment (start 124 94) (end 122.25 92.25) (width 0.8) (layer "F.Cu") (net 1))
 (segment (start 135.75 94.5) (end 127.75 94.5) (width 0.8) (layer "F.Cu") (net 1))
 (segment (start 134.25 89.25) (end 137 89.25) (width 0.5) (layer "F.Cu") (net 5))
 (segment (start 137 89.25) (end 138 90.25) (width 0.5) (layer "F.Cu") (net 5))
 (segment (start 131.675 89) (end 132.375 88.3) (width 0.5) (layer "F.Cu") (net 3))
 (segment (start 129.95 89) (end 131.675 89) (width 0.5) (layer "F.Cu") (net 3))
 (segment (start 127.25 86.25) (end 127 86) (width 0.5) (layer "F.Cu") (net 6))
 (segment (start 127.75 86) (end 125.5 86) (width 0.5) (layer "F.Cu") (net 6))
 (segment (start 125.5 86) (end 125 86.5) (width 0.5) (layer "F.Cu") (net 6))
 (segment (start 127.25 88.05) (end 127.25 86.25) (width 0.5) (layer "F.Cu") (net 6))
 (segment (start 129.95 88.05) (end 129.95 86.2) (width 0.5) (layer "F.Cu") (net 7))
 (segment (start 132 86) (end 132.25 86.25) (width 0.5) (layer "F.Cu") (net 7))
 (segment (start 129.95 86.2) (end 129.75 86) (width 0.5) (layer "F.Cu") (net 7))
 (segment (start 129.75 86) (end 132 86) (width 0.5) (layer "F.Cu") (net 7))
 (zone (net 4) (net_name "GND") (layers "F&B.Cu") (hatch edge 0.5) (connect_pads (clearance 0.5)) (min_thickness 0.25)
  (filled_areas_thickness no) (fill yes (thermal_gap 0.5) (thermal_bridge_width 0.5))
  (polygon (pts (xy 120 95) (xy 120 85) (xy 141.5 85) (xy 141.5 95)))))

